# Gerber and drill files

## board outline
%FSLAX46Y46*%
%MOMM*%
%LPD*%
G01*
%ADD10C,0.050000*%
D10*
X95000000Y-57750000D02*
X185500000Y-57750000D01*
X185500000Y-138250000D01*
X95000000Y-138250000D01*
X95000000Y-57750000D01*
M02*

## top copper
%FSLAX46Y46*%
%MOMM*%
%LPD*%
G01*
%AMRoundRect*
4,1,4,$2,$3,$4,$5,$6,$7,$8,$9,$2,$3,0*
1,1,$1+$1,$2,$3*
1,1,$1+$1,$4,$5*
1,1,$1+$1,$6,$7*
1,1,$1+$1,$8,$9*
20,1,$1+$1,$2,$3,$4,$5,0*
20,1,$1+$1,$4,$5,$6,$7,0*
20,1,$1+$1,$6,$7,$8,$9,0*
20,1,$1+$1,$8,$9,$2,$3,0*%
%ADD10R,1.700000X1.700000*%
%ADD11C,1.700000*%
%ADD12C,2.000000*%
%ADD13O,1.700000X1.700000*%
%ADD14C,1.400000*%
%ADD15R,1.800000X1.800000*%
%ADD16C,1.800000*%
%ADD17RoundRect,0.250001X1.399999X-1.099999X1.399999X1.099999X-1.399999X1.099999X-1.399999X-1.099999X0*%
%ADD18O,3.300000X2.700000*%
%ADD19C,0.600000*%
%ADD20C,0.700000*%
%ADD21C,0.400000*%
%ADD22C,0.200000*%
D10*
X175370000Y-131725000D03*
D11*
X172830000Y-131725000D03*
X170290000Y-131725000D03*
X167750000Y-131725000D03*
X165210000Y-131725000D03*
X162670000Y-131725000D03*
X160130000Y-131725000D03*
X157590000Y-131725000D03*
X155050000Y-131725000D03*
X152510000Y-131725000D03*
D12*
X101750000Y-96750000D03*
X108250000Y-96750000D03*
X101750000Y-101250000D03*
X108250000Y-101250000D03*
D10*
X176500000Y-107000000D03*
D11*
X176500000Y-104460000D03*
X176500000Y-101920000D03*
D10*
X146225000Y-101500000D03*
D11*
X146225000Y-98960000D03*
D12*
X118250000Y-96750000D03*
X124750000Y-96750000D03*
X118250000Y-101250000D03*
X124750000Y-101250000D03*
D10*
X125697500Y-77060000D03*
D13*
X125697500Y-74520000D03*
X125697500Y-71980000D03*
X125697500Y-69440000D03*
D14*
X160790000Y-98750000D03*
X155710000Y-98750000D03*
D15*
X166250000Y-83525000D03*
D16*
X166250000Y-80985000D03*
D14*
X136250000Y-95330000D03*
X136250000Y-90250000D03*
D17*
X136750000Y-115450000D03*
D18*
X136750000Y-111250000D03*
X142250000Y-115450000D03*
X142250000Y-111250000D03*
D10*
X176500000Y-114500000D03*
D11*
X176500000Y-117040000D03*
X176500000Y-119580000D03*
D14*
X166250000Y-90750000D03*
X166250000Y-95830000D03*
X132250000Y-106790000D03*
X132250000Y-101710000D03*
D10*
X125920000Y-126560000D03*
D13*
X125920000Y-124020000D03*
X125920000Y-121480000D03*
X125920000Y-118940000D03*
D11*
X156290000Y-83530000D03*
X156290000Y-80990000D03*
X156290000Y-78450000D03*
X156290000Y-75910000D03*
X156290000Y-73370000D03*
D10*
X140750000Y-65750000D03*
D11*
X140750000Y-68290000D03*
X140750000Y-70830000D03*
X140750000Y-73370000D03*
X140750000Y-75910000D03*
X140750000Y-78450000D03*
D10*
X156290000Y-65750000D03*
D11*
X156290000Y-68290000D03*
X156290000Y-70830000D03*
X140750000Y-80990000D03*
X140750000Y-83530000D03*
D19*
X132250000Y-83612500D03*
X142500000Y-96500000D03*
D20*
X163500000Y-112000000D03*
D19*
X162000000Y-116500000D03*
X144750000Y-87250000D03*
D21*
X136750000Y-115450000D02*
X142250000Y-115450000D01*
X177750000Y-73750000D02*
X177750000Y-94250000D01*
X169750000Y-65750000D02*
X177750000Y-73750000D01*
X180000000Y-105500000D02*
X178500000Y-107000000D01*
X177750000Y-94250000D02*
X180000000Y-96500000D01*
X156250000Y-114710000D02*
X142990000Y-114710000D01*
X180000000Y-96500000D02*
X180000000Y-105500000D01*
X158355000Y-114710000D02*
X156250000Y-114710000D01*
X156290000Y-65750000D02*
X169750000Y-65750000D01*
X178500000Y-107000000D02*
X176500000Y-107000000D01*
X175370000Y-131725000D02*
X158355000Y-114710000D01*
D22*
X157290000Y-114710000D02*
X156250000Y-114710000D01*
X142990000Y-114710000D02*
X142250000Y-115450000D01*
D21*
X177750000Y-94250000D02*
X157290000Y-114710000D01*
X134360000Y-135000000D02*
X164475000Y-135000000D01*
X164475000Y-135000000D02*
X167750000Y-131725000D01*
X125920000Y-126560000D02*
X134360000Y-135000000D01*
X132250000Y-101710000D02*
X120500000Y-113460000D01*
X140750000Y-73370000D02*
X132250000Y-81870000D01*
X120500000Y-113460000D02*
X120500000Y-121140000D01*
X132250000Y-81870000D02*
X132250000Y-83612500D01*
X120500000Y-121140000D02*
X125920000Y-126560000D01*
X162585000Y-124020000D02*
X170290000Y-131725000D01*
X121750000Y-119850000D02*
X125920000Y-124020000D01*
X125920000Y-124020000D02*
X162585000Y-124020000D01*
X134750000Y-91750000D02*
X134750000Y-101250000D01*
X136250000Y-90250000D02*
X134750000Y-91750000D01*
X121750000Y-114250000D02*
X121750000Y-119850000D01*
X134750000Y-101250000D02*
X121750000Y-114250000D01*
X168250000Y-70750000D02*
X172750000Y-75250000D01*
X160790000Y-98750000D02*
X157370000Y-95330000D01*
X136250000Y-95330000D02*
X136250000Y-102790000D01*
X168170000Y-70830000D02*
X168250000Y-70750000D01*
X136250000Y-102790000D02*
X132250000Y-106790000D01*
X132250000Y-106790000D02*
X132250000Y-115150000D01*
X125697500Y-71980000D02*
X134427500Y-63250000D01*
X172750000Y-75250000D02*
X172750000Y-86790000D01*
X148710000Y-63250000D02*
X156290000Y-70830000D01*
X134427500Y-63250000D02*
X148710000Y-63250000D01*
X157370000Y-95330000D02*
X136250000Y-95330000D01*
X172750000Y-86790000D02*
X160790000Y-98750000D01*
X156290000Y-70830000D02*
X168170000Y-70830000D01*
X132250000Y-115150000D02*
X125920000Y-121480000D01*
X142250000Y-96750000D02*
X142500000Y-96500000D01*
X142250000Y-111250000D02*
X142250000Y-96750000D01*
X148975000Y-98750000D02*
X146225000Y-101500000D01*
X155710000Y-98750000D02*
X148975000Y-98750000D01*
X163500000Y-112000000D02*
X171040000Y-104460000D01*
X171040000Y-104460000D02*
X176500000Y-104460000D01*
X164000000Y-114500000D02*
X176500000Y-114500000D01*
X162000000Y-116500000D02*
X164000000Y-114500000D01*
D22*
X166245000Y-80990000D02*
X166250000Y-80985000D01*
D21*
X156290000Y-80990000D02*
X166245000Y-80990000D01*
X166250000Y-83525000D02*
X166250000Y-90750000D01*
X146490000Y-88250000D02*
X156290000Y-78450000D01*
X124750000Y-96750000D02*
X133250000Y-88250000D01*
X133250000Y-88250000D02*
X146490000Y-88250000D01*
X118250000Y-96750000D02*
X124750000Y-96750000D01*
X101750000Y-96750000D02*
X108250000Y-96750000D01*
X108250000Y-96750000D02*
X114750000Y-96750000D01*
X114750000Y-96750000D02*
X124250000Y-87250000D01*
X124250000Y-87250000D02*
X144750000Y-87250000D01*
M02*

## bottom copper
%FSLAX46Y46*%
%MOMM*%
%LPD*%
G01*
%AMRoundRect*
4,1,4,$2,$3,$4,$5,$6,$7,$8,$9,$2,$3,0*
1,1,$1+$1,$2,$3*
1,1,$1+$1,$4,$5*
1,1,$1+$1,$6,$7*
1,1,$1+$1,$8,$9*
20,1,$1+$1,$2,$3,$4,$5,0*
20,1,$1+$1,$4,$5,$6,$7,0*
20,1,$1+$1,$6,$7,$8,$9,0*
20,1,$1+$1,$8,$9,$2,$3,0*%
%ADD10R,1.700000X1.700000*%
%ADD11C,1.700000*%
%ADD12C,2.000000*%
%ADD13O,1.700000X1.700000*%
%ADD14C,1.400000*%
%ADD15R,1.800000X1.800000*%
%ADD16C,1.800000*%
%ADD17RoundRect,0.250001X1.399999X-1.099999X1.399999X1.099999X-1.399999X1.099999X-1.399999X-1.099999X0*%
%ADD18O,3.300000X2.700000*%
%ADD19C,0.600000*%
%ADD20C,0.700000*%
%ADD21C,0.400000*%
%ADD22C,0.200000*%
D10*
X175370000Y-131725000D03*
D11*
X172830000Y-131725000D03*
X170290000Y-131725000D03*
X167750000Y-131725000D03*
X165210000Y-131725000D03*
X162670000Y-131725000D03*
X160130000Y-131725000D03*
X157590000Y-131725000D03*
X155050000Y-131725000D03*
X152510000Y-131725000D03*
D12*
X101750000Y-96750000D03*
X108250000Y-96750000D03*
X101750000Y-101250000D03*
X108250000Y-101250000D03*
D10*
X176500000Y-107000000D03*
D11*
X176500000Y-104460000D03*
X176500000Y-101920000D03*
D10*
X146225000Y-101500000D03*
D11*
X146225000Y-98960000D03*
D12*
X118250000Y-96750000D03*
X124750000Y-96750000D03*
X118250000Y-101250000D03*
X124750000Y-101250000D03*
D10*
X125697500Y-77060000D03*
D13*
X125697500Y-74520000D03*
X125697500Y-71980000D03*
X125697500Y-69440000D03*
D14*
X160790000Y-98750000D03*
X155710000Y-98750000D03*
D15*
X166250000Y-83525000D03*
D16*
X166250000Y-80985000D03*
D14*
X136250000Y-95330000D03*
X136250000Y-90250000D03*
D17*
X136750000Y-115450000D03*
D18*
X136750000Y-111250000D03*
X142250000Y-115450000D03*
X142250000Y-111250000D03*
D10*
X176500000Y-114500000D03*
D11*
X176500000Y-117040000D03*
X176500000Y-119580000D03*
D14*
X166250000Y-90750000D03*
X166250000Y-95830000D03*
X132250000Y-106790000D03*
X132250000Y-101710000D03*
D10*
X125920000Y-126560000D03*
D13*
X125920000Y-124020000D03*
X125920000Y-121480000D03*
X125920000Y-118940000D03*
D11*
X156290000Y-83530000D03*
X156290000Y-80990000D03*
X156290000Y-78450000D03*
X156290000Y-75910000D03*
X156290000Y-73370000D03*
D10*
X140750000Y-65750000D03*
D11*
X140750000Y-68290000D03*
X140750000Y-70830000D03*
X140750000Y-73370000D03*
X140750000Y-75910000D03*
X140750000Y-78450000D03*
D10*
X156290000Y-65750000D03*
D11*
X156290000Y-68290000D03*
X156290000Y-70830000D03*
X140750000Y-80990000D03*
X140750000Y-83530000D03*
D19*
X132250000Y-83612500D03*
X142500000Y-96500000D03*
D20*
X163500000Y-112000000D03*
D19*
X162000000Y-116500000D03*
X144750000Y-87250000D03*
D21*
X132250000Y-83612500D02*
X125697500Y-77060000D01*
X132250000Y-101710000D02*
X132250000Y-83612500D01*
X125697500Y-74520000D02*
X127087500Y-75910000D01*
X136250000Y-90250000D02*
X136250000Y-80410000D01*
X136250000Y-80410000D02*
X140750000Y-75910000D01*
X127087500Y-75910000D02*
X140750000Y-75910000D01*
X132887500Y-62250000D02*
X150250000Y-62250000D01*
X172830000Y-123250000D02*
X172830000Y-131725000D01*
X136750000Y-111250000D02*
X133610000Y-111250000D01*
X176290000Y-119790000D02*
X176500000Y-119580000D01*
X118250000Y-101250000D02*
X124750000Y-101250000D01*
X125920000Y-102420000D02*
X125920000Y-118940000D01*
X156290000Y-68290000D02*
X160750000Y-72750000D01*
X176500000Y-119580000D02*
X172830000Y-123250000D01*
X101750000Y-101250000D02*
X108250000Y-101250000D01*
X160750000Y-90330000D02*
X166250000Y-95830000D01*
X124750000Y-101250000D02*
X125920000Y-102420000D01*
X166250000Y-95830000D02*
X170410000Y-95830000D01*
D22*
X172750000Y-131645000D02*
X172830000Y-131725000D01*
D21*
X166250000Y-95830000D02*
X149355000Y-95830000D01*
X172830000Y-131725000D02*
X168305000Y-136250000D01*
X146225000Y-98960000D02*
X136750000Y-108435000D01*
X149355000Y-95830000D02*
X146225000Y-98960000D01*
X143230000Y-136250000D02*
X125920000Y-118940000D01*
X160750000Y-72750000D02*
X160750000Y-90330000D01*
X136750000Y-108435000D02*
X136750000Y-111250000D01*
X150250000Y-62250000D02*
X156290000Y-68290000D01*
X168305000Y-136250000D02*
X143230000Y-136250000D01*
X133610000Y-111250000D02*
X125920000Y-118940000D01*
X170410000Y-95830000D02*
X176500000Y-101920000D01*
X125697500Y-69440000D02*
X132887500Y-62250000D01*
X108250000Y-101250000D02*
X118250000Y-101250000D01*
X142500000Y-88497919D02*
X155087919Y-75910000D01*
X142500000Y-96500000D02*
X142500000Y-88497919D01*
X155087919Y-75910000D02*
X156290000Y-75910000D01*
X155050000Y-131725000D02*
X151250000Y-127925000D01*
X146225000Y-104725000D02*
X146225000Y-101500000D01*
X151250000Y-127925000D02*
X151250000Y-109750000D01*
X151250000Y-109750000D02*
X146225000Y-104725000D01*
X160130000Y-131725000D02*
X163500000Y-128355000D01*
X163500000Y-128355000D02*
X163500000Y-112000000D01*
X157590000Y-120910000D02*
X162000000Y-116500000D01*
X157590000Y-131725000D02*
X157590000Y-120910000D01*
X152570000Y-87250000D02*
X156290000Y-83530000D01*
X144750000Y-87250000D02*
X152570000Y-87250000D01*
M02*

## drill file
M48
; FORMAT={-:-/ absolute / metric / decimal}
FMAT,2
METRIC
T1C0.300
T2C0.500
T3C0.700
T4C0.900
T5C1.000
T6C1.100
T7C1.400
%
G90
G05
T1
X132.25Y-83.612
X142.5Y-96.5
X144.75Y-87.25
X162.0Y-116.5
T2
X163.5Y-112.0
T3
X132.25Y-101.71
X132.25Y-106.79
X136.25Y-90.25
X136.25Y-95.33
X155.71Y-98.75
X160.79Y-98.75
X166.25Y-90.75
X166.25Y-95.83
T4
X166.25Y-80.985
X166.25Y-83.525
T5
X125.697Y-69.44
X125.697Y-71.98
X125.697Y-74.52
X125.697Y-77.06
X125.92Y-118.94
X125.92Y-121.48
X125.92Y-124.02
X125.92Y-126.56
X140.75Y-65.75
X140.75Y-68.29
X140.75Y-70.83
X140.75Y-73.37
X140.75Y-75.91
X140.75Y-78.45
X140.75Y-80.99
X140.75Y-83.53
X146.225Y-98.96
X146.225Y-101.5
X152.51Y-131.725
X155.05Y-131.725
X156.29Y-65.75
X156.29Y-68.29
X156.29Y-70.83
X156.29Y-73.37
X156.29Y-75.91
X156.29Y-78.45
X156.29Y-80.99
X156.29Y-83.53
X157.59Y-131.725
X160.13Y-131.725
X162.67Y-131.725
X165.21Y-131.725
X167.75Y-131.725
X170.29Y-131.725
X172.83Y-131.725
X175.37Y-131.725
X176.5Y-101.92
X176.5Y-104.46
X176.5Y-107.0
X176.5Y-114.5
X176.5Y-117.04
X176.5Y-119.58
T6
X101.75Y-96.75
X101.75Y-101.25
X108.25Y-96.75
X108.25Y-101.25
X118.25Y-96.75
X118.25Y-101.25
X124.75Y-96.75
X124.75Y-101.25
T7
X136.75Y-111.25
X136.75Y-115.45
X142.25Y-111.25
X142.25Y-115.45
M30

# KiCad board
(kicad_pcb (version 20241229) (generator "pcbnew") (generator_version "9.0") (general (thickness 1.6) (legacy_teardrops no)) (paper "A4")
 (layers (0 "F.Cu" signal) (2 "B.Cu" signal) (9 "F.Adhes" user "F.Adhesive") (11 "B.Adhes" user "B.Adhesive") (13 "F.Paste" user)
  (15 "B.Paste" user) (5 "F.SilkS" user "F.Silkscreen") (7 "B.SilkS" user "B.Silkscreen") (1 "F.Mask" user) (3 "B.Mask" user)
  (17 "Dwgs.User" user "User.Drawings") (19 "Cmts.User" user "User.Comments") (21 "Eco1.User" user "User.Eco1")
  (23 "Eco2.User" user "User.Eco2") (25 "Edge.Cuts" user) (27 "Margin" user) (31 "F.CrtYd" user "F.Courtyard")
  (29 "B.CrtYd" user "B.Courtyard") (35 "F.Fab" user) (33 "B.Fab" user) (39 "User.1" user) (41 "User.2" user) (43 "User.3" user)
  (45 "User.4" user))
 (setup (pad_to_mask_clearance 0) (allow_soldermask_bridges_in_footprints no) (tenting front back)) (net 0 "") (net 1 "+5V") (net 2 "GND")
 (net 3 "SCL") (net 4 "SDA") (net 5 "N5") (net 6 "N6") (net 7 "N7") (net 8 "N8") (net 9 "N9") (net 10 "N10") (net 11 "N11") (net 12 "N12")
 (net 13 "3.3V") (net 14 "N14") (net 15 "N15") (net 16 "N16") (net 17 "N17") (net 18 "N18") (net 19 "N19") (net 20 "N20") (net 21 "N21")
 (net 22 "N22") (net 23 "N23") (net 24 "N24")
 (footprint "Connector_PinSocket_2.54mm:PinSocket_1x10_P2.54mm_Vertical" (layer "F.Cu") (at 175.37 131.725 -90)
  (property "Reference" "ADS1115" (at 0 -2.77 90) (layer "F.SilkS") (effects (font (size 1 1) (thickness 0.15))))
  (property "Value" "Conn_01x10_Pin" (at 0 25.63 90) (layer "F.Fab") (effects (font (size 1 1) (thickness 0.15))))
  (pad "1" thru_hole rect (at 0 0 270) (size 1.7 1.7) (drill 1) (layers "*.Cu" "*.Mask") (remove_unused_layers no) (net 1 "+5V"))
  (pad "2" thru_hole circle (at 0 2.54 270) (size 1.7 1.7) (drill 1) (layers "*.Cu" "*.Mask") (remove_unused_layers no) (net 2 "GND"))
  (pad "3" thru_hole circle (at 0 5.08 270) (size 1.7 1.7) (drill 1) (layers "*.Cu" "*.Mask") (remove_unused_layers no) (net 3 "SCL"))
  (pad "4" thru_hole circle (at 0 7.62 270) (size 1.7 1.7) (drill 1) (layers "*.Cu" "*.Mask") (remove_unused_layers no) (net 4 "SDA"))
  (pad "5" thru_hole circle (at 0 10.16 270) (size 1.7 1.7) (drill 1) (layers "*.Cu" "*.Mask") (remove_unused_layers no) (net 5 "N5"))
  (pad "6" thru_hole circle (at 0 12.7 270) (size 1.7 1.7) (drill 1) (layers "*.Cu" "*.Mask") (remove_unused_layers no) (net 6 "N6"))
  (pad "7" thru_hole circle (at 0 15.24 270) (size 1.7 1.7) (drill 1) (layers "*.Cu" "*.Mask") (remove_unused_layers no) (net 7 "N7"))
  (pad "8" thru_hole circle (at 0 17.78 270) (size 1.7 1.7) (drill 1) (layers "*.Cu" "*.Mask") (remove_unused_layers no) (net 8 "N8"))
  (pad "9" thru_hole circle (at 0 20.32 270) (size 1.7 1.7) (drill 1) (layers "*.Cu" "*.Mask") (remove_unused_layers no) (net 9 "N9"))
  (pad "10" thru_hole circle (at 0 22.86 270) (size 1.7 1.7) (drill 1) (layers "*.Cu" "*.Mask") (remove_unused_layers no) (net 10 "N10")))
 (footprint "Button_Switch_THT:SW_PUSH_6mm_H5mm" (layer "F.Cu") (at 101.75 96.75)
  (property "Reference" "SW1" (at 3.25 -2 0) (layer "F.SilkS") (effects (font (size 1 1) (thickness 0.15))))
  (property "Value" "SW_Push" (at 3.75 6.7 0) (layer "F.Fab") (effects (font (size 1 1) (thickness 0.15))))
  (pad "1" thru_hole circle (at 0 0 90) (size 2 2) (drill 1.1) (layers "*.Cu" "*.Mask") (remove_unused_layers no) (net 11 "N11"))
  (pad "1" thru_hole circle (at 6.5 0 90) (size 2 2) (drill 1.1) (layers "*.Cu" "*.Mask") (remove_unused_layers no) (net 11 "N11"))
  (pad "2" thru_hole circle (at 0 4.5 90) (size 2 2) (drill 1.1) (layers "*.Cu" "*.Mask") (remove_unused_layers no) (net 2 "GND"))
  (pad "2" thru_hole circle (at 6.5 4.5 90) (size 2 2) (drill 1.1) (layers "*.Cu" "*.Mask") (remove_unused_layers no) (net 2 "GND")))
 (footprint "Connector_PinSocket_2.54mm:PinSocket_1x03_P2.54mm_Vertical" (layer "F.Cu") (at 176.5 107 180)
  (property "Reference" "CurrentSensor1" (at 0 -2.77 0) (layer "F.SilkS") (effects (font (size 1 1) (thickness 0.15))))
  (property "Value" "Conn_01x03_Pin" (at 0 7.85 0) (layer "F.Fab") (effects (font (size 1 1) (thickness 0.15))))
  (pad "1" thru_hole rect (at 0 0 180) (size 1.7 1.7) (drill 1) (layers "*.Cu" "*.Mask") (remove_unused_layers no) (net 1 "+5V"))
  (pad "2" thru_hole circle (at 0 2.54 180) (size 1.7 1.7) (drill 1) (layers "*.Cu" "*.Mask") (remove_unused_layers no) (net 7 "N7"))
  (pad "3" thru_hole circle (at 0 5.08 180) (size 1.7 1.7) (drill 1) (layers "*.Cu" "*.Mask") (remove_unused_layers no) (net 2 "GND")))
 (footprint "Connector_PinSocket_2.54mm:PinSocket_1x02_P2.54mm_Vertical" (layer "F.Cu") (at 146.225 101.5 180)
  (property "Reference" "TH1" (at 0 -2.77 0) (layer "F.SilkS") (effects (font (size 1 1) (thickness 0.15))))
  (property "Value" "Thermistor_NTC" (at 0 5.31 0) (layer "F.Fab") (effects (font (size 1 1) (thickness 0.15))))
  (pad "1" thru_hole rect (at 0 0 180) (size 1.7 1.7) (drill 1) (layers "*.Cu" "*.Mask") (remove_unused_layers no) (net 9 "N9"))
  (pad "2" thru_hole circle (at 0 2.54 180) (size 1.7 1.7) (drill 1) (layers "*.Cu" "*.Mask") (remove_unused_layers no) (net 2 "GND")))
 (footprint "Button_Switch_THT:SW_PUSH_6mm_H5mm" (layer "F.Cu") (at 118.25 96.75)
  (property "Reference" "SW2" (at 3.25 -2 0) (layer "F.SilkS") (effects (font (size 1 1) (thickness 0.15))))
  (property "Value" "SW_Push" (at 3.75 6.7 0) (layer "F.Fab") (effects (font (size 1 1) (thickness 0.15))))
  (pad "1" thru_hole circle (at 0 0 90) (size 2 2) (drill 1.1) (layers "*.Cu" "*.Mask") (remove_unused_layers no) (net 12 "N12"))
  (pad "1" thru_hole circle (at 6.5 0 90) (size 2 2) (drill 1.1) (layers "*.Cu" "*.Mask") (remove_unused_layers no) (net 12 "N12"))
  (pad "2" thru_hole circle (at 0 4.5 90) (size 2 2) (drill 1.1) (layers "*.Cu" "*.Mask") (remove_unused_layers no) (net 2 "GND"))
  (pad "2" thru_hole circle (at 6.5 4.5 90) (size 2 2) (drill 1.1) (layers "*.Cu" "*.Mask") (remove_unused_layers no) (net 2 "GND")))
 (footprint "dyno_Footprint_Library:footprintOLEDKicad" (layer "F.Cu") (at 124.5275 68.25)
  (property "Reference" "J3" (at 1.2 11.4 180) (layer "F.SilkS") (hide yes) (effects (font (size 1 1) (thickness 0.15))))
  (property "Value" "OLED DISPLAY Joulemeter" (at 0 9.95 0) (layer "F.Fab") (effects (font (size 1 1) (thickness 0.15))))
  (pad "1" thru_hole rect (at 1.17 8.81 180) (size 1.7 1.7) (drill 1) (layers "*.Cu" "*.Mask") (remove_unused_layers no) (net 4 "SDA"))
  (pad "2" thru_hole oval (at 1.17 6.27 180) (size 1.7 1.7) (drill 1) (layers "*.Cu" "*.Mask") (remove_unused_layers no) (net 3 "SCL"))
  (pad "3" thru_hole oval (at 1.17 3.73 180) (size 1.7 1.7) (drill 1) (layers "*.Cu" "*.Mask") (remove_unused_layers no) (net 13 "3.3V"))
  (pad "4" thru_hole oval (at 1.17 1.19 180) (size 1.7 1.7) (drill 1) (layers "*.Cu" "*.Mask") (remove_unused_layers no) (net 2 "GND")))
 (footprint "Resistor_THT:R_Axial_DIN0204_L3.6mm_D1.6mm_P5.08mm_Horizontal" (layer "F.Cu") (at 160.79 98.75 180)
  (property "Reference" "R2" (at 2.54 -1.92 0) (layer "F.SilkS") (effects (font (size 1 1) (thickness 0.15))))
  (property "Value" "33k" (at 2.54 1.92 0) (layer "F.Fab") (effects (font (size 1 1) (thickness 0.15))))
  (pad "1" thru_hole circle (at 0 0 180) (size 1.4 1.4) (drill 0.7) (layers "*.Cu" "*.Mask") (remove_unused_layers no) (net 13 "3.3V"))
  (pad "2" thru_hole circle (at 5.08 0 180) (size 1.4 1.4) (drill 0.7) (layers "*.Cu" "*.Mask") (remove_unused_layers no) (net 9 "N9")))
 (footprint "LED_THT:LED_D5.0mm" (layer "F.Cu") (at 166.25 83.525 90)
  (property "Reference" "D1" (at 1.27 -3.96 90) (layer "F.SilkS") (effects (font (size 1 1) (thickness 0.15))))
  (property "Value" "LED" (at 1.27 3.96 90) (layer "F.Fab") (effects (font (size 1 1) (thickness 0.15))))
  (pad "1" thru_hole rect (at 0 0 90) (size 1.8 1.8) (drill 0.9) (layers "*.Cu" "*.Mask") (remove_unused_layers no) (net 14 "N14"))
  (pad "2" thru_hole circle (at 2.54 0 90) (size 1.8 1.8) (drill 0.9) (layers "*.Cu" "*.Mask") (remove_unused_layers no) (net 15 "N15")))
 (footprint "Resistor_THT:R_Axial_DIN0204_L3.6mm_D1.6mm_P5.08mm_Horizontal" (layer "F.Cu") (at 136.25 95.33 90)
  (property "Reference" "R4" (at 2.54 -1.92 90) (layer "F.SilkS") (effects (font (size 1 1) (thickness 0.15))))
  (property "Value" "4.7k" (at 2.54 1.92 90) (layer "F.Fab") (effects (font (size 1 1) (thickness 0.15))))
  (pad "1" thru_hole circle (at 0 0 90) (size 1.4 1.4) (drill 0.7) (layers "*.Cu" "*.Mask") (remove_unused_layers no) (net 13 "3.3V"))
  (pad "2" thru_hole circle (at 5.08 0 90) (size 1.4 1.4) (drill 0.7) (layers "*.Cu" "*.Mask") (remove_unused_layers no) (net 3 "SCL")))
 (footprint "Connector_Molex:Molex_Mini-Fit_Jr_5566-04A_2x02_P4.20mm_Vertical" (layer "F.Cu") (at 136.75 115.45 90)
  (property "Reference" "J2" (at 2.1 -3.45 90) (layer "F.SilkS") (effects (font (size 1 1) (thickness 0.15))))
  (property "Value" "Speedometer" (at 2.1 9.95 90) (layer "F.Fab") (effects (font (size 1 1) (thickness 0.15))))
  (pad "1" thru_hole roundrect (at 0 0 90) (size 2.7 3.3) (drill 1.4) (layers "*.Cu" "*.Mask") (remove_unused_layers no)
   (roundrect_rratio 0.092593) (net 1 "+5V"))
  (pad "2" thru_hole oval (at 4.2 0 90) (size 2.7 3.3) (drill 1.4) (layers "*.Cu" "*.Mask") (remove_unused_layers no) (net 2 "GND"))
  (pad "3" thru_hole oval (at 0 5.5 90) (size 2.7 3.3) (drill 1.4) (layers "*.Cu" "*.Mask") (remove_unused_layers no) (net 1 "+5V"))
  (pad "4" thru_hole oval (at 4.2 5.5 90) (size 2.7 3.3) (drill 1.4) (layers "*.Cu" "*.Mask") (remove_unused_layers no) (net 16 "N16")))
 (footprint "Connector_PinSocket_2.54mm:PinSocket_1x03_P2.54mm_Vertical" (layer "F.Cu") (at 176.5 114.5)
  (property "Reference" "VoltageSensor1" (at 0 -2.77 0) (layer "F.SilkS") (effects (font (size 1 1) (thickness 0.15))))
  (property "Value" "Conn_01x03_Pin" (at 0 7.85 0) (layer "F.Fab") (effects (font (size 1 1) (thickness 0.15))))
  (pad "1" thru_hole rect (at 0 0) (size 1.7 1.7) (drill 1) (layers "*.Cu" "*.Mask") (remove_unused_layers no) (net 8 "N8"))
  (pad "2" thru_hole circle (at 0 2.54) (size 1.7 1.7) (drill 1) (layers "*.Cu" "*.Mask") (remove_unused_layers no) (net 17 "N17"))
  (pad "3" thru_hole circle (at 0 5.08) (size 1.7 1.7) (drill 1) (layers "*.Cu" "*.Mask") (remove_unused_layers no) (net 2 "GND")))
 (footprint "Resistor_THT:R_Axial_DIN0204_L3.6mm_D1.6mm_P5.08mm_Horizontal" (layer "F.Cu") (at 166.25 90.75 -90)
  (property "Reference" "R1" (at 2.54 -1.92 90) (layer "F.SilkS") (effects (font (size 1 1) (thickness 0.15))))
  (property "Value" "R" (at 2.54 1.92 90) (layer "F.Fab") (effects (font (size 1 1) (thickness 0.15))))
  (pad "1" thru_hole circle (at 0 0 270) (size 1.4 1.4) (drill 0.7) (layers "*.Cu" "*.Mask") (remove_unused_layers no) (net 14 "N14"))
  (pad "2" thru_hole circle (at 5.08 0 270) (size 1.4 1.4) (drill 0.7) (layers "*.Cu" "*.Mask") (remove_unused_layers no) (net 2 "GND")))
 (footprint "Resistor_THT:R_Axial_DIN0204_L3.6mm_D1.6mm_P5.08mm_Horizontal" (layer "F.Cu") (at 132.25 106.79 90)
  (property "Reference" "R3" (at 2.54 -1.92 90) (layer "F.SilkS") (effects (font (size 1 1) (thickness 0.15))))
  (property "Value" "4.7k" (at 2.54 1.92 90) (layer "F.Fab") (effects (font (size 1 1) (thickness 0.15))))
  (pad "1" thru_hole circle (at 0 0 90) (size 1.4 1.4) (drill 0.7) (layers "*.Cu" "*.Mask") (remove_unused_layers no) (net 13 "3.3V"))
  (pad "2" thru_hole circle (at 5.08 0 90) (size 1.4 1.4) (drill 0.7) (layers "*.Cu" "*.Mask") (remove_unused_layers no) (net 4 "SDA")))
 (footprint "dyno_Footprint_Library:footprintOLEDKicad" (layer "F.Cu") (at 124.75 117.75)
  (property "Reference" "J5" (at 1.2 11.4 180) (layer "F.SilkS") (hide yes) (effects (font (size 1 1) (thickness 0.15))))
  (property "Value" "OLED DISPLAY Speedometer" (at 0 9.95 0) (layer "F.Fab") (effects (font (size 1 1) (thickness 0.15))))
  (pad "1" thru_hole rect (at 1.17 8.81 180) (size 1.7 1.7) (drill 1) (layers "*.Cu" "*.Mask") (remove_unused_layers no) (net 4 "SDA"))
  (pad "2" thru_hole oval (at 1.17 6.27 180) (size 1.7 1.7) (drill 1) (layers "*.Cu" "*.Mask") (remove_unused_layers no) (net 3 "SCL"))
  (pad "3" thru_hole oval (at 1.17 3.73 180) (size 1.7 1.7) (drill 1) (layers "*.Cu" "*.Mask") (remove_unused_layers no) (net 13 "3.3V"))
  (pad "4" thru_hole oval (at 1.17 1.19 180) (size 1.7 1.7) (drill 1) (layers "*.Cu" "*.Mask") (remove_unused_layers no) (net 2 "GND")))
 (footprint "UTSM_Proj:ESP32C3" (layer "F.Cu") (at 148.52 74.8)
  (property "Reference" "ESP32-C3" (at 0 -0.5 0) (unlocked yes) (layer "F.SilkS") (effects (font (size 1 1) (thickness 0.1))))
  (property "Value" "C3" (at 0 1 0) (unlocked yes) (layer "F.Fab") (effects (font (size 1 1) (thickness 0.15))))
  (pad "0" thru_hole circle (at 7.77 8.73) (size 1.7 1.7) (drill 1) (layers "*.Cu" "*.Mask") (remove_unused_layers no) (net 11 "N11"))
  (pad "1" thru_hole circle (at 7.77 6.19) (size 1.7 1.7) (drill 1) (layers "*.Cu" "*.Mask") (remove_unused_layers no) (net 15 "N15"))
  (pad "2" thru_hole circle (at 7.77 3.65) (size 1.7 1.7) (drill 1) (layers "*.Cu" "*.Mask") (remove_unused_layers no) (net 12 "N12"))
  (pad "3" thru_hole circle (at 7.77 1.11) (size 1.7 1.7) (drill 1) (layers "*.Cu" "*.Mask") (remove_unused_layers no) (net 16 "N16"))
  (pad "4" thru_hole circle (at 7.77 -1.43) (size 1.7 1.7) (drill 1) (layers "*.Cu" "*.Mask") (remove_unused_layers no) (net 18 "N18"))
  (pad "5" thru_hole rect (at -7.77 -9.05) (size 1.7 1.7) (drill 1) (layers "*.Cu" "*.Mask") (remove_unused_layers no) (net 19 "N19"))
  (pad "6" thru_hole circle (at -7.77 -6.51) (size 1.7 1.7) (drill 1) (layers "*.Cu" "*.Mask") (remove_unused_layers no) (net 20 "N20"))
  (pad "7" thru_hole circle (at -7.77 -3.97) (size 1.7 1.7) (drill 1) (layers "*.Cu" "*.Mask") (remove_unused_layers no) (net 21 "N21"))
  (pad "8" thru_hole circle (at -7.77 -1.43) (size 1.7 1.7) (drill 1) (layers "*.Cu" "*.Mask") (remove_unused_layers no) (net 4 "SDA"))
  (pad "9" thru_hole circle (at -7.77 1.11) (size 1.7 1.7) (drill 1) (layers "*.Cu" "*.Mask") (remove_unused_layers no) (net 3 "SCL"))
  (pad "10" thru_hole circle (at -7.77 3.65) (size 1.7 1.7) (drill 1) (layers "*.Cu" "*.Mask") (remove_unused_layers no) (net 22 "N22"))
  (pad "11" thru_hole rect (at 7.77 -9.05) (size 1.7 1.7) (drill 1) (layers "*.Cu" "*.Mask") (remove_unused_layers no) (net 1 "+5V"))
  (pad "12" thru_hole circle (at 7.77 -6.51) (size 1.7 1.7) (drill 1) (layers "*.Cu" "*.Mask") (remove_unused_layers no) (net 2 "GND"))
  (pad "13" thru_hole circle (at 7.77 -3.97) (size 1.7 1.7) (drill 1) (layers "*.Cu" "*.Mask") (remove_unused_layers no) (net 13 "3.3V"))
  (pad "20" thru_hole circle (at -7.77 6.19) (size 1.7 1.7) (drill 1) (layers "*.Cu" "*.Mask") (remove_unused_layers no) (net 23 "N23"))
  (pad "21" thru_hole circle (at -7.77 8.73) (size 1.7 1.7) (drill 1) (layers "*.Cu" "*.Mask") (remove_unused_layers no) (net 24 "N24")))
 (gr_rect (start 95 57.75) (end 185.5 138.25) (stroke (width 0.05) (type solid)) (fill no) (layer "Edge.Cuts"))
 (segment (start 136.75 115.45) (end 142.25 115.45) (width 0.4) (layer "F.Cu") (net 1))
 (segment (start 177.75 73.75) (end 177.75 94.25) (width 0.4) (layer "F.Cu") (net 1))
 (segment (start 169.75 65.75) (end 177.75 73.75) (width 0.4) (layer "F.Cu") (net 1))
 (segment (start 180 105.5) (end 178.5 107) (width 0.4) (layer "F.Cu") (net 1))
 (segment (start 177.75 94.25) (end 180 96.5) (width 0.4) (layer "F.Cu") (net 1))
 (segment (start 156.25 114.71) (end 142.99 114.71) (width 0.4) (layer "F.Cu") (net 1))
 (segment (start 180 96.5) (end 180 105.5) (width 0.4) (layer "F.Cu") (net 1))
 (segment (start 158.355 114.71) (end 156.25 114.71) (width 0.4) (layer "F.Cu") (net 1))
 (segment (start 156.29 65.75) (end 169.75 65.75) (width 0.4) (layer "F.Cu") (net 1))
 (segment (start 178.5 107) (end 176.5 107) (width 0.4) (layer "F.Cu") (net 1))
 (segment (start 175.37 131.725) (end 158.355 114.71) (width 0.4) (layer "F.Cu") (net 1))
 (segment (start 157.29 114.71) (end 156.25 114.71) (width 0.2) (layer "F.Cu") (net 1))
 (segment (start 142.99 114.71) (end 142.25 115.45) (width 0.2) (layer "F.Cu") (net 1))
 (segment (start 177.75 94.25) (end 157.29 114.71) (width 0.4) (layer "F.Cu") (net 1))
 (segment (start 134.36 135) (end 164.475 135) (width 0.4) (layer "F.Cu") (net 4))
 (segment (start 164.475 135) (end 167.75 131.725) (width 0.4) (layer "F.Cu") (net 4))
 (segment (start 125.92 126.56) (end 134.36 135) (width 0.4) (layer "F.Cu") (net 4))
 (segment (start 132.25 101.71) (end 120.5 113.46) (width 0.4) (layer "F.Cu") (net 4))
 (segment (start 140.75 73.37) (end 132.25 81.87) (width 0.4) (layer "F.Cu") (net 4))
 (segment (start 120.5 113.46) (end 120.5 121.14) (width 0.4) (layer "F.Cu") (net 4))
 (segment (start 132.25 81.87) (end 132.25 83.6125) (width 0.4) (layer "F.Cu") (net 4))
 (segment (start 120.5 121.14) (end 125.92 126.56) (width 0.4) (layer "F.Cu") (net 4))
 (via (at 132.25 83.6125) (size 0.6) (drill 0.3) (layers "F.Cu" "B.Cu") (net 4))
 (segment (start 132.25 83.6125) (end 125.6975 77.06) (width 0.4) (layer "B.Cu") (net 4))
 (segment (start 132.25 101.71) (end 132.25 83.6125) (width 0.4) (layer "B.Cu") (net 4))
 (segment (start 162.585 124.02) (end 170.29 131.725) (width 0.4) (layer "F.Cu") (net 3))
 (segment (start 121.75 119.85) (end 125.92 124.02) (width 0.4) (layer "F.Cu") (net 3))
 (segment (start 125.92 124.02) (end 162.585 124.02) (width 0.4) (layer "F.Cu") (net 3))
 (segment (start 134.75 91.75) (end 134.75 101.25) (width 0.4) (layer "F.Cu") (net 3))
 (segment (start 136.25 90.25) (end 134.75 91.75) (width 0.4) (layer "F.Cu") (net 3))
 (segment (start 121.75 114.25) (end 121.75 119.85) (width 0.4) (layer "F.Cu") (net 3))
 (segment (start 134.75 101.25) (end 121.75 114.25) (width 0.4) (layer "F.Cu") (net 3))
 (segment (start 125.6975 74.52) (end 127.0875 75.91) (width 0.4) (layer "B.Cu") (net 3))
 (segment (start 136.25 90.25) (end 136.25 80.41) (width 0.4) (layer "B.Cu") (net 3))
 (segment (start 136.25 80.41) (end 140.75 75.91) (width 0.4) (layer "B.Cu") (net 3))
 (segment (start 127.0875 75.91) (end 140.75 75.91) (width 0.4) (layer "B.Cu") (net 3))
 (segment (start 132.8875 62.25) (end 150.25 62.25) (width 0.4) (layer "B.Cu") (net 2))
 (segment (start 172.83 123.25) (end 172.83 131.725) (width 0.4) (layer "B.Cu") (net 2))
 (segment (start 136.75 111.25) (end 133.61 111.25) (width 0.4) (layer "B.Cu") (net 2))
 (segment (start 176.29 119.79) (end 176.5 119.58) (width 0.4) (layer "B.Cu") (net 2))
 (segment (start 118.25 101.25) (end 124.75 101.25) (width 0.4) (layer "B.Cu") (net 2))
 (segment (start 125.92 102.42) (end 125.92 118.94) (width 0.4) (layer "B.Cu") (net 2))
 (segment (start 156.29 68.29) (end 160.75 72.75) (width 0.4) (layer "B.Cu") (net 2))
 (segment (start 176.5 119.58) (end 172.83 123.25) (width 0.4) (layer "B.Cu") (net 2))
 (segment (start 101.75 101.25) (end 108.25 101.25) (width 0.4) (layer "B.Cu") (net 2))
 (segment (start 160.75 90.33) (end 166.25 95.83) (width 0.4) (layer "B.Cu") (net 2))
 (segment (start 124.75 101.25) (end 125.92 102.42) (width 0.4) (layer "B.Cu") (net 2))
 (segment (start 166.25 95.83) (end 170.41 95.83) (width 0.4) (layer "B.Cu") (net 2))
 (segment (start 172.75 131.645) (end 172.83 131.725) (width 0.2) (layer "B.Cu") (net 2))
 (segment (start 166.25 95.83) (end 149.355 95.83) (width 0.4) (layer "B.Cu") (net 2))
 (segment (start 172.83 131.725) (end 168.305 136.25) (width 0.4) (layer "B.Cu") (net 2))
 (segment (start 146.225 98.96) (end 136.75 108.435) (width 0.4) (layer "B.Cu") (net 2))
 (segment (start 149.355 95.83) (end 146.225 98.96) (width 0.4) (layer "B.Cu") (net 2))
 (segment (start 143.23 136.25) (end 125.92 118.94) (width 0.4) (layer "B.Cu") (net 2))
 (segment (start 160.75 72.75) (end 160.75 90.33) (width 0.4) (layer "B.Cu") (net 2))
 (segment (start 136.75 108.435) (end 136.75 111.25) (width 0.4) (layer "B.Cu") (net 2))
 (segment (start 150.25 62.25) (end 156.29 68.29) (width 0.4) (layer "B.Cu") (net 2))
 (segment (start 168.305 136.25) (end 143.23 136.25) (width 0.4) (layer "B.Cu") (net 2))
 (segment (start 133.61 111.25) (end 125.92 118.94) (width 0.4) (layer "B.Cu") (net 2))
 (segment (start 170.41 95.83) (end 176.5 101.92) (width 0.4) (layer "B.Cu") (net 2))
 (segment (start 125.6975 69.44) (end 132.8875 62.25) (width 0.4) (layer "B.Cu") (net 2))
 (segment (start 108.25 101.25) (end 118.25 101.25) (width 0.4) (layer "B.Cu") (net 2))
 (segment (start 168.25 70.75) (end 172.75 75.25) (width 0.4) (layer "F.Cu") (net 13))
 (segment (start 160.79 98.75) (end 157.37 95.33) (width 0.4) (layer "F.Cu") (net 13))
 (segment (start 136.25 95.33) (end 136.25 102.79) (width 0.4) (layer "F.Cu") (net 13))
 (segment (start 168.17 70.83) (end 168.25 70.75) (width 0.4) (layer "F.Cu") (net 13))
 (segment (start 136.25 102.79) (end 132.25 106.79) (width 0.4) (layer "F.Cu") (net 13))
 (segment (start 132.25 106.79) (end 132.25 115.15) (width 0.4) (layer "F.Cu") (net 13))
 (segment (start 125.6975 71.98) (end 134.4275 63.25) (width 0.4) (layer "F.Cu") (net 13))
 (segment (start 172.75 75.25) (end 172.75 86.79) (width 0.4) (layer "F.Cu") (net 13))
 (segment (start 148.71 63.25) (end 156.29 70.83) (width 0.4) (layer "F.Cu") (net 13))
 (segment (start 134.4275 63.25) (end 148.71 63.25) (width 0.4) (layer "F.Cu") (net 13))
 (segment (start 157.37 95.33) (end 136.25 95.33) (width 0.4) (layer "F.Cu") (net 13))
 (segment (start 172.75 86.79) (end 160.79 98.75) (width 0.4) (layer "F.Cu") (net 13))
 (segment (start 156.29 70.83) (end 168.17 70.83) (width 0.4) (layer "F.Cu") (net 13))
 (segment (start 132.25 115.15) (end 125.92 121.48) (width 0.4) (layer "F.Cu") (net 13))
 (segment (start 142.25 96.75) (end 142.5 96.5) (width 0.4) (layer "F.Cu") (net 16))
 (segment (start 142.25 111.25) (end 142.25 96.75) (width 0.4) (layer "F.Cu") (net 16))
 (via (at 142.5 96.5) (size 0.6) (drill 0.3) (layers "F.Cu" "B.Cu") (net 16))
 (segment (start 142.5 88.497919) (end 155.087919 75.91) (width 0.4) (layer "B.Cu") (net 16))
 (segment (start 142.5 96.5) (end 142.5 88.497919) (width 0.4) (layer "B.Cu") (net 16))
 (segment (start 155.087919 75.91) (end 156.29 75.91) (width 0.4) (layer "B.Cu") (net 16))
 (segment (start 148.975 98.75) (end 146.225 101.5) (width 0.4) (layer "F.Cu") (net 9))
 (segment (start 155.71 98.75) (end 148.975 98.75) (width 0.4) (layer "F.Cu") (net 9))
 (segment (start 155.05 131.725) (end 151.25 127.925) (width 0.4) (layer "B.Cu") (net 9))
 (segment (start 146.225 104.725) (end 146.225 101.5) (width 0.4) (layer "B.Cu") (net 9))
 (segment (start 151.25 127.925) (end 151.25 109.75) (width 0.4) (layer "B.Cu") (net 9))
 (segment (start 151.25 109.75) (end 146.225 104.725) (width 0.4) (layer "B.Cu") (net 9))
 (segment (start 163.5 112) (end 171.04 104.46) (width 0.4) (layer "F.Cu") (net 7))
 (segment (start 171.04 104.46) (end 176.5 104.46) (width 0.4) (layer "F.Cu") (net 7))
 (via (at 163.5 112) (size 0.7) (drill 0.5) (layers "F.Cu" "B.Cu") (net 7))
 (segment (start 160.13 131.725) (end 163.5 128.355) (width 0.4) (layer "B.Cu") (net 7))
 (segment (start 163.5 128.355) (end 163.5 112) (width 0.4) (layer "B.Cu") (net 7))
 (segment (start 164 114.5) (end 176.5 114.5) (width 0.4) (layer "F.Cu") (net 8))
 (segment (start 162 116.5) (end 164 114.5) (width 0.4) (layer "F.Cu") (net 8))
 (via (at 162 116.5) (size 0.6) (drill 0.3) (layers "F.Cu" "B.Cu") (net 8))
 (segment (start 157.59 120.91) (end 162 116.5) (width 0.4) (layer "B.Cu") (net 8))
 (segment (start 157.59 131.725) (end 157.59 120.91) (width 0.4) (layer "B.Cu") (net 8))
 (segment (start 166.245 80.99) (end 166.25 80.985) (width 0.2) (layer "F.Cu") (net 15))
 (segment (start 156.29 80.99) (end 166.245 80.99) (width 0.4) (layer "F.Cu") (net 15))
 (segment (start 166.25 83.525) (end 166.25 90.75) (width 0.4) (layer "F.Cu") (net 14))
 (segment (start 146.49 88.25) (end 156.29 78.45) (width 0.4) (layer "F.Cu") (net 12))
 (segment (start 124.75 96.75) (end 133.25 88.25) (width 0.4) (layer "F.Cu") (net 12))
 (segment (start 133.25 88.25) (end 146.49 88.25) (width 0.4) (layer "F.Cu") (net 12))
 (segment (start 118.25 96.75) (end 124.75 96.75) (width 0.4) (layer "F.Cu") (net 12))
 (segment (start 101.75 96.75) (end 108.25 96.75) (width 0.4) (layer "F.Cu") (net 11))
 (segment (start 108.25 96.75) (end 114.75 96.75) (width 0.4) (layer "F.Cu") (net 11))
 (segment (start 114.75 96.75) (end 124.25 87.25) (width 0.4) (layer "F.Cu") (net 11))
 (segment (start 124.25 87.25) (end 144.75 87.25) (width 0.4) (layer "F.Cu") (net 11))
 (via (at 144.75 87.25) (size 0.6) (drill 0.3) (layers "F.Cu" "B.Cu") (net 11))
 (segment (start 152.57 87.25) (end 156.29 83.53) (width 0.4) (layer "B.Cu") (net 11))
 (segment (start 144.75 87.25) (end 152.57 87.25) (width 0.4) (layer "B.Cu") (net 11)))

